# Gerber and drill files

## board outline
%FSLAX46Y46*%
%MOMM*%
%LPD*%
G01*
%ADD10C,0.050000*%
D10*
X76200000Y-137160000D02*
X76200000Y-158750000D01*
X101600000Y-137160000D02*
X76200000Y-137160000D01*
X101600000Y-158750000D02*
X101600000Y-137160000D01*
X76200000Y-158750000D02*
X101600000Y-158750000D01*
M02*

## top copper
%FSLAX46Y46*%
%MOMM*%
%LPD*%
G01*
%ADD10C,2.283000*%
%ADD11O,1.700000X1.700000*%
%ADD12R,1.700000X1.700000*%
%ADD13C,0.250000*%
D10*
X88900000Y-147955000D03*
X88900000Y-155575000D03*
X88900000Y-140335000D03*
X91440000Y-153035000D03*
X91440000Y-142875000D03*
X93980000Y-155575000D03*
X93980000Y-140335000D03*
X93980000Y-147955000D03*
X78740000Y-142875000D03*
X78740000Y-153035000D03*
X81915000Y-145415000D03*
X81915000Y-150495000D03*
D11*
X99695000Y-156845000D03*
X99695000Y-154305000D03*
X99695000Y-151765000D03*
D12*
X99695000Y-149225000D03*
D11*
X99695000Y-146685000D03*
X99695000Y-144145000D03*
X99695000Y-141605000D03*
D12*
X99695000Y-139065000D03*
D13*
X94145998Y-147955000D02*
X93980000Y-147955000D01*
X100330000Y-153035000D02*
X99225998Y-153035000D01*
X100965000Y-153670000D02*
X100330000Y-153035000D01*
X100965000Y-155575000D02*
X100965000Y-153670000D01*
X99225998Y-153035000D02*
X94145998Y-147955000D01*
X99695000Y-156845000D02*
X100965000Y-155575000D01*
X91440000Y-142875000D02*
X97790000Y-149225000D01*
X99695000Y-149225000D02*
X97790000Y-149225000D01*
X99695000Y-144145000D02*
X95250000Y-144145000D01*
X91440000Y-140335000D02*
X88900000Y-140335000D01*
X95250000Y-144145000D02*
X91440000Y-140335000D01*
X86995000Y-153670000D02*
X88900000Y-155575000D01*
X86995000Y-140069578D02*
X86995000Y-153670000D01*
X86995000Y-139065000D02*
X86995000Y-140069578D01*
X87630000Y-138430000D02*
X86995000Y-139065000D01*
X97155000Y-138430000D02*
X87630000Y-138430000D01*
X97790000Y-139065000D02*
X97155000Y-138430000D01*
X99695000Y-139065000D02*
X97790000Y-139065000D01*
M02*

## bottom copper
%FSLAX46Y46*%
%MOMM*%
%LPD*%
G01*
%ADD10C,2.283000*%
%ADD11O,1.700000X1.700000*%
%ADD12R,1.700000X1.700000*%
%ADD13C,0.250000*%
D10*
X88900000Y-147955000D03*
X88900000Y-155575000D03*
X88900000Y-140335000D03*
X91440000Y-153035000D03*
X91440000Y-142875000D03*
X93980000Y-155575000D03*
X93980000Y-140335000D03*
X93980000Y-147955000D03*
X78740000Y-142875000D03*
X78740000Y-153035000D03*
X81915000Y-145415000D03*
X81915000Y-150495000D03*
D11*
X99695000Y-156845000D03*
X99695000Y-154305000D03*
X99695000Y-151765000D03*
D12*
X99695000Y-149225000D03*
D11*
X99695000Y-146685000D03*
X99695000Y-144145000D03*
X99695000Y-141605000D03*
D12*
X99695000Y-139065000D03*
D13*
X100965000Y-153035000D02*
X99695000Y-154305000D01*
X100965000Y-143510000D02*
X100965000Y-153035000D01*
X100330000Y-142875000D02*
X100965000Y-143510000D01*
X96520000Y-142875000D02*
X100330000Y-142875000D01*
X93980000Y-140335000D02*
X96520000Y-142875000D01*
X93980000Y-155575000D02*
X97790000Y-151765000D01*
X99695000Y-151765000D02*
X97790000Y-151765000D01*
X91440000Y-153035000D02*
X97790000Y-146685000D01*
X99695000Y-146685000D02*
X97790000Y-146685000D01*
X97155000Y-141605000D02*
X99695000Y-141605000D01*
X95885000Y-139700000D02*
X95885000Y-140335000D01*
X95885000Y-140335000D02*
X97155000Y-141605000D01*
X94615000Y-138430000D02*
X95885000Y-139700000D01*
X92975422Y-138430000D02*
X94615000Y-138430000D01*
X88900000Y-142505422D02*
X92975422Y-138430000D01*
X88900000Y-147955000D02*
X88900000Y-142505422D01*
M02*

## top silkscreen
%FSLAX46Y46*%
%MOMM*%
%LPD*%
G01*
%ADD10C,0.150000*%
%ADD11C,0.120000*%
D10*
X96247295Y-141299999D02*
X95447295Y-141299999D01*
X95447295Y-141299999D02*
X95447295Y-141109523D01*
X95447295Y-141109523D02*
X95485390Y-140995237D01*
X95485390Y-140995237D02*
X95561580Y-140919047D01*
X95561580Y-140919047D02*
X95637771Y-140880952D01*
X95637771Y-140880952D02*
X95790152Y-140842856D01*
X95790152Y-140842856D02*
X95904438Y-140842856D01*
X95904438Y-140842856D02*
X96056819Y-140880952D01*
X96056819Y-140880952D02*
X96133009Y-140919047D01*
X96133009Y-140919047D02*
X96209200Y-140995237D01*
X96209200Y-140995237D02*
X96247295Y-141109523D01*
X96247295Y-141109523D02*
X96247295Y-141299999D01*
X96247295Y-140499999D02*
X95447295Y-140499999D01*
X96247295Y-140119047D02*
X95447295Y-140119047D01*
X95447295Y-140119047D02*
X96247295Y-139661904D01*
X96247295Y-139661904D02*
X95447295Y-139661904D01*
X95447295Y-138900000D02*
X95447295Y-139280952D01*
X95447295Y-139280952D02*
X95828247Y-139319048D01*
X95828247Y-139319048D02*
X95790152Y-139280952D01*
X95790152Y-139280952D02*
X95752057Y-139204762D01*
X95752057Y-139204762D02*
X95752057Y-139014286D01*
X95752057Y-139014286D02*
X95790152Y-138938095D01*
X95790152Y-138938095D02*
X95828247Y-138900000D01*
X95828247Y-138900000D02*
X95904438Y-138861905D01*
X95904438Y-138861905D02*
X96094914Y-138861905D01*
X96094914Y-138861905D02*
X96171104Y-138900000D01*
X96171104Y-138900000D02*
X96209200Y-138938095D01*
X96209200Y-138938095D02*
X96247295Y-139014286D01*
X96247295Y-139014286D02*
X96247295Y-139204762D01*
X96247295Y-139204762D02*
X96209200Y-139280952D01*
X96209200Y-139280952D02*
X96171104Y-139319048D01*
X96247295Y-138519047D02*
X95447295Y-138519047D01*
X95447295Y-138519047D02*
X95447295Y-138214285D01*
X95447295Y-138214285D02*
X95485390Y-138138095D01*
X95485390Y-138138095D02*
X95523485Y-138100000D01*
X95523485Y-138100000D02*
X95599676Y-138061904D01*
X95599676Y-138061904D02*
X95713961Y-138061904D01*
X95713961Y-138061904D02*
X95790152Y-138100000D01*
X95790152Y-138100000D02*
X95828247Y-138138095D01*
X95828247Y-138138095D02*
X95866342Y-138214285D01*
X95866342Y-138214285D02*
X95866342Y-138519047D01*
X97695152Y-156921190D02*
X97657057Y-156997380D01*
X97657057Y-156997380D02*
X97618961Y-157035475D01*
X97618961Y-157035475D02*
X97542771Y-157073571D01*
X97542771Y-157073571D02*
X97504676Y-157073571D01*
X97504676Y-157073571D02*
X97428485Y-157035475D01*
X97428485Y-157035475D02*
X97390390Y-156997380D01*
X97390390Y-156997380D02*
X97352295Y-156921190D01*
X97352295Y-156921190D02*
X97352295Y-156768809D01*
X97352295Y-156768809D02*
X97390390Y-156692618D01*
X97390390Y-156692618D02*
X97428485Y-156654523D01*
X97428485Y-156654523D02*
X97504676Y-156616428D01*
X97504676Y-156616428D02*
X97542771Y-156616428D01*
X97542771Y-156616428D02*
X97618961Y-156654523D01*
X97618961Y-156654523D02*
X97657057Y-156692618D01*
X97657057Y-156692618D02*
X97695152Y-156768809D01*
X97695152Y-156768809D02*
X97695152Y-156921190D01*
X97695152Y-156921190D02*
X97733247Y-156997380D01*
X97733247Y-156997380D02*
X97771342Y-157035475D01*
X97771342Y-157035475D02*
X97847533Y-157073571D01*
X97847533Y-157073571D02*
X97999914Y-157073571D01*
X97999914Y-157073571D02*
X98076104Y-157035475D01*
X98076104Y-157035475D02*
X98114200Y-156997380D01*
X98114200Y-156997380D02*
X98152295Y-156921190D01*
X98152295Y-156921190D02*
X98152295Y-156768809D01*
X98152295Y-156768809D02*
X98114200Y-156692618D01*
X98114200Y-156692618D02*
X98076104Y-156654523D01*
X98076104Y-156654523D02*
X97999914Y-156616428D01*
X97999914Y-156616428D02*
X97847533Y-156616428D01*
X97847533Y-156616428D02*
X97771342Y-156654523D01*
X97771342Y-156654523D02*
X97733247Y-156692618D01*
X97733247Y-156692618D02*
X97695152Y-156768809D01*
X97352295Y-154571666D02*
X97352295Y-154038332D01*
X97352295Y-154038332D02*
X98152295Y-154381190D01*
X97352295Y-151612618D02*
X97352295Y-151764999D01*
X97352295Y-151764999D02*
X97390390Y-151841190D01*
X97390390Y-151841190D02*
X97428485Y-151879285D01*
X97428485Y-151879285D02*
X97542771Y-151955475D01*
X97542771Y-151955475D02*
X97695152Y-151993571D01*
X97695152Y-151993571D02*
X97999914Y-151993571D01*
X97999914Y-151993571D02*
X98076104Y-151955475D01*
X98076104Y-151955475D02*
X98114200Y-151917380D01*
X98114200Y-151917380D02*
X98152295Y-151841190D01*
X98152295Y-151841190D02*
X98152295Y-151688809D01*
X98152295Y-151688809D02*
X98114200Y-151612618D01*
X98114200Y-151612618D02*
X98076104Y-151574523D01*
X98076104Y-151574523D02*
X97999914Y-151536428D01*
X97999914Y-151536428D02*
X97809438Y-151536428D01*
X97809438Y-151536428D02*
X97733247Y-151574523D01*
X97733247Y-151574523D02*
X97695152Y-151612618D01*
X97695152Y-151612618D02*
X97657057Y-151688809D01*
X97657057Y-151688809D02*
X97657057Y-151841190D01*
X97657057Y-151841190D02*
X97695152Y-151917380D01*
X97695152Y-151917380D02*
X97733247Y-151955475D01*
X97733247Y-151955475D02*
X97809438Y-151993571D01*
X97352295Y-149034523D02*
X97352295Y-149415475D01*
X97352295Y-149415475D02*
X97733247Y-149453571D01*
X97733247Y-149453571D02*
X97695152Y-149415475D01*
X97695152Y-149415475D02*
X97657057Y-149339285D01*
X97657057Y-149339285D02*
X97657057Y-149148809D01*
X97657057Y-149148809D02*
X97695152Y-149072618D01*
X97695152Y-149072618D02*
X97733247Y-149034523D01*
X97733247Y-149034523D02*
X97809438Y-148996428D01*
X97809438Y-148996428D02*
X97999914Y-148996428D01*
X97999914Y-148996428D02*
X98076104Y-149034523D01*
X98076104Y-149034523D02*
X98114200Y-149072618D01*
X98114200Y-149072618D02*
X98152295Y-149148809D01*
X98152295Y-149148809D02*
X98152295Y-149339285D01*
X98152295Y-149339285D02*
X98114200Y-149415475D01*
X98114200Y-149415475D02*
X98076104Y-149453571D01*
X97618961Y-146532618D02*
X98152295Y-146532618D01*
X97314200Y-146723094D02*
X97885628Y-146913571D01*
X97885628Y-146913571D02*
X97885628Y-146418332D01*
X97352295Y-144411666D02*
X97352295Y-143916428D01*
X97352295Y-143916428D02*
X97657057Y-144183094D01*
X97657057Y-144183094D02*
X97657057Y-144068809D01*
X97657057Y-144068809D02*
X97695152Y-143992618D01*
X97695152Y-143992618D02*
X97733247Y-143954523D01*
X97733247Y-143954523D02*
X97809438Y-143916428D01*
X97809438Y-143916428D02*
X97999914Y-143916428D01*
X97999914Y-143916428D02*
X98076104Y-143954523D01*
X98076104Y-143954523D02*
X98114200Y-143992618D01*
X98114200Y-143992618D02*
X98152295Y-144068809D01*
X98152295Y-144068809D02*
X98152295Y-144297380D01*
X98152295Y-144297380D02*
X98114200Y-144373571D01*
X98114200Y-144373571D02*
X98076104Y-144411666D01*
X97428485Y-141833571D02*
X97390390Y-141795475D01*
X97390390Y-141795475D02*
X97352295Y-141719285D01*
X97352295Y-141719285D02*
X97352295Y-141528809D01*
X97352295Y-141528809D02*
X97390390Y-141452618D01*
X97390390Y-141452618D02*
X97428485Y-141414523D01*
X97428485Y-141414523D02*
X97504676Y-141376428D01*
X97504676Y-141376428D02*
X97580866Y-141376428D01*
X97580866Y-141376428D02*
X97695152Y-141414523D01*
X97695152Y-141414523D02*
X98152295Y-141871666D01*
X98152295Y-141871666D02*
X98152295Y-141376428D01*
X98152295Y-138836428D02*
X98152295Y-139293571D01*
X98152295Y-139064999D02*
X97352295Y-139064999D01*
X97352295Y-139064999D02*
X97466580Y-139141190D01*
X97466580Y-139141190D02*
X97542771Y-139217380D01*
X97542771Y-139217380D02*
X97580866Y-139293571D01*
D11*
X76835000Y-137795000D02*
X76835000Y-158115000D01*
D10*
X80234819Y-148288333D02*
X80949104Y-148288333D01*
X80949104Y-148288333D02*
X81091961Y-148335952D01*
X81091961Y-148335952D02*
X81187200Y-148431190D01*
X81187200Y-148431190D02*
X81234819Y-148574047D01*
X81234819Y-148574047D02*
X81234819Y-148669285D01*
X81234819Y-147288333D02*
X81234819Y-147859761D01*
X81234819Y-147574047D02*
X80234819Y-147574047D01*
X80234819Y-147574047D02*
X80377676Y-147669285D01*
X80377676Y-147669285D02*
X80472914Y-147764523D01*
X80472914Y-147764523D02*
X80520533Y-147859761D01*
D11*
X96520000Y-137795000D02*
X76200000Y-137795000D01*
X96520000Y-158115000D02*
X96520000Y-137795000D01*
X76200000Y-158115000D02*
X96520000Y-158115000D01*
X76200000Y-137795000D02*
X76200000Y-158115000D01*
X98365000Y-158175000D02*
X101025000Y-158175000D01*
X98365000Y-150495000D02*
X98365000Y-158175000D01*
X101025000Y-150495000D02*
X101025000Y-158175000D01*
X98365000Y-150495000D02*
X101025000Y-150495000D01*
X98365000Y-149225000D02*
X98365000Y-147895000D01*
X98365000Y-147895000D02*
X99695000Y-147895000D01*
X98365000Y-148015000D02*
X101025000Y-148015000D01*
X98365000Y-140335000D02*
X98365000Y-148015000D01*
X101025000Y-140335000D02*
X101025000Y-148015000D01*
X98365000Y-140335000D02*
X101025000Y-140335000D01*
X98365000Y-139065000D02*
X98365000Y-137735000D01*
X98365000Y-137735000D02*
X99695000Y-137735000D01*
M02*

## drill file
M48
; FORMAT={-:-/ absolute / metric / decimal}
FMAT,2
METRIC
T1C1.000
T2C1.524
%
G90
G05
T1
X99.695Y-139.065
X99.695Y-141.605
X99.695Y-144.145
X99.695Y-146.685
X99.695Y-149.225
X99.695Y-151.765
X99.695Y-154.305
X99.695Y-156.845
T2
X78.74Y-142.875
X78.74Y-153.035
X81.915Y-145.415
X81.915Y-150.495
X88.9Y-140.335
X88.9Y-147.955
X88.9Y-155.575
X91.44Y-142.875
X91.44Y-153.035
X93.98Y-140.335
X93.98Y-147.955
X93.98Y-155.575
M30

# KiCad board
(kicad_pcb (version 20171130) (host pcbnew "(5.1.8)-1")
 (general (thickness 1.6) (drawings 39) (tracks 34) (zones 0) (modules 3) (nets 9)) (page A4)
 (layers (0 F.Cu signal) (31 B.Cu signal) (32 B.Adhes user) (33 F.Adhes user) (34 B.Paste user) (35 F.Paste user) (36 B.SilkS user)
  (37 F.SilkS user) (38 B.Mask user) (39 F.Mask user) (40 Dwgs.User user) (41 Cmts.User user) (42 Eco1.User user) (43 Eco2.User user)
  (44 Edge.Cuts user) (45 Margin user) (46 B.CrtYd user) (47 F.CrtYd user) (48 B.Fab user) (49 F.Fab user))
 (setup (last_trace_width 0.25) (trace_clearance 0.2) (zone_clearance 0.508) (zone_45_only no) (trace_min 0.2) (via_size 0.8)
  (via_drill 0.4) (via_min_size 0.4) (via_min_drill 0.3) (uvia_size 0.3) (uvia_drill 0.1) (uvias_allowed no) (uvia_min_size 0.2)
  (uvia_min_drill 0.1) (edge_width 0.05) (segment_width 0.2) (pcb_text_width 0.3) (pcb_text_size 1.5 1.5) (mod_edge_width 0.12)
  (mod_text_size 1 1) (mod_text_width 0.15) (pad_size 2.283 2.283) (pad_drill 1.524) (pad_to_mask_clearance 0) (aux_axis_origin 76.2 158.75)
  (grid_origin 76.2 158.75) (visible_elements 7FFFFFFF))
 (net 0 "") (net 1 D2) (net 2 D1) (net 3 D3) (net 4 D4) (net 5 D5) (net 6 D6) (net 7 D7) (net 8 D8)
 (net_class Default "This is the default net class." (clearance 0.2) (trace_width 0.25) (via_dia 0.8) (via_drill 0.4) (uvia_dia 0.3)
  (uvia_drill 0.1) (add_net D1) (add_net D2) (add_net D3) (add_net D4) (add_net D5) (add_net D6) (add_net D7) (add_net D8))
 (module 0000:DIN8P (layer F.Cu) (at 81.28 147.955 270)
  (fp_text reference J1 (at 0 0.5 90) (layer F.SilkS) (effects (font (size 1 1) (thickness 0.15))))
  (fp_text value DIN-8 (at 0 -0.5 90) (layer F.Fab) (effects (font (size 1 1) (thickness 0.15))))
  (fp_line (start -10.16 -15.24) (end -10.16 5.08) (layer F.SilkS) (width 0.12))
  (fp_line (start 10.16 -15.24) (end -10.16 -15.24) (layer F.SilkS) (width 0.12))
  (fp_line (start 10.16 5.08) (end 10.16 -15.24) (layer F.SilkS) (width 0.12))
  (fp_line (start -10.16 5.08) (end 10.16 5.08) (layer F.SilkS) (width 0.12))
  (pad 2 thru_hole circle (at 0 -7.62 270) (size 2.283 2.283) (drill 1.524) (layers *.Cu *.Mask) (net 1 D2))
  (pad 1 thru_hole circle (at 7.62 -7.62 270) (size 2.283 2.283) (drill 1.524) (layers *.Cu *.Mask) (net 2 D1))
  (pad 3 thru_hole circle (at -7.62 -7.62 270) (size 2.283 2.283) (drill 1.524) (layers *.Cu *.Mask) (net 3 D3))
  (pad 4 thru_hole circle (at 5.08 -10.16 270) (size 2.283 2.283) (drill 1.524) (layers *.Cu *.Mask) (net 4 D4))
  (pad 5 thru_hole circle (at -5.08 -10.16 270) (size 2.283 2.283) (drill 1.524) (layers *.Cu *.Mask) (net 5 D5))
  (pad 6 thru_hole circle (at 7.62 -12.7 270) (size 2.283 2.283) (drill 1.524) (layers *.Cu *.Mask) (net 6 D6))
  (pad 7 thru_hole circle (at -7.62 -12.7 270) (size 2.283 2.283) (drill 1.524) (layers *.Cu *.Mask) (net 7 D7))
  (pad 8 thru_hole circle (at 0 -12.7 270) (size 2.283 2.283) (drill 1.524) (layers *.Cu *.Mask) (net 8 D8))
  (pad "" thru_hole circle (at -5.08 2.54 270) (size 2.283 2.283) (drill 1.524) (layers *.Cu *.Mask))
  (pad "" thru_hole circle (at 5.08 2.54 270) (size 2.283 2.283) (drill 1.524) (layers *.Cu *.Mask))
  (pad "" thru_hole circle (at -2.54 -0.635 270) (size 2.283 2.283) (drill 1.524) (layers *.Cu *.Mask))
  (pad "" thru_hole circle (at 2.54 -0.635 270) (size 2.283 2.283) (drill 1.524) (layers *.Cu *.Mask)))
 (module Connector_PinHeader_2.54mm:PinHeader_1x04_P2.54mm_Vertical (layer F.Cu) (at 99.695 149.225)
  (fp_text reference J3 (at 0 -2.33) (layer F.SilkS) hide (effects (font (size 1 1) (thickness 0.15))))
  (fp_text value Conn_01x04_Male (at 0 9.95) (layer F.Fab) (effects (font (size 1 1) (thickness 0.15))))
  (fp_line (start -1.33 8.95) (end 1.33 8.95) (layer F.SilkS) (width 0.12))
  (fp_line (start -1.33 1.27) (end -1.33 8.95) (layer F.SilkS) (width 0.12))
  (fp_line (start 1.33 1.27) (end 1.33 8.95) (layer F.SilkS) (width 0.12))
  (fp_line (start -1.33 1.27) (end 1.33 1.27) (layer F.SilkS) (width 0.12))
  (fp_line (start -1.33 0) (end -1.33 -1.33) (layer F.SilkS) (width 0.12))
  (fp_line (start -1.33 -1.33) (end 0 -1.33) (layer F.SilkS) (width 0.12))
  (pad 4 thru_hole oval (at 0 7.62) (size 1.7 1.7) (drill 1) (layers *.Cu *.Mask) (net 8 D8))
  (pad 3 thru_hole oval (at 0 5.08) (size 1.7 1.7) (drill 1) (layers *.Cu *.Mask) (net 7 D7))
  (pad 2 thru_hole oval (at 0 2.54) (size 1.7 1.7) (drill 1) (layers *.Cu *.Mask) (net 6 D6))
  (pad 1 thru_hole rect (at 0 0) (size 1.7 1.7) (drill 1) (layers *.Cu *.Mask) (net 5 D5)))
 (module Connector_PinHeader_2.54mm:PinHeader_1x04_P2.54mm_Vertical (layer F.Cu) (at 99.695 139.065)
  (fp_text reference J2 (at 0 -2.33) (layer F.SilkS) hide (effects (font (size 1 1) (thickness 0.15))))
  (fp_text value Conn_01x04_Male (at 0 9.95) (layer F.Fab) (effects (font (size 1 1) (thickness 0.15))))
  (fp_line (start -1.33 8.95) (end 1.33 8.95) (layer F.SilkS) (width 0.12))
  (fp_line (start -1.33 1.27) (end -1.33 8.95) (layer F.SilkS) (width 0.12))
  (fp_line (start 1.33 1.27) (end 1.33 8.95) (layer F.SilkS) (width 0.12))
  (fp_line (start -1.33 1.27) (end 1.33 1.27) (layer F.SilkS) (width 0.12))
  (fp_line (start -1.33 0) (end -1.33 -1.33) (layer F.SilkS) (width 0.12))
  (fp_line (start -1.33 -1.33) (end 0 -1.33) (layer F.SilkS) (width 0.12))
  (pad 4 thru_hole oval (at 0 7.62) (size 1.7 1.7) (drill 1) (layers *.Cu *.Mask) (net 4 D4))
  (pad 3 thru_hole oval (at 0 5.08) (size 1.7 1.7) (drill 1) (layers *.Cu *.Mask) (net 3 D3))
  (pad 2 thru_hole oval (at 0 2.54) (size 1.7 1.7) (drill 1) (layers *.Cu *.Mask) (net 1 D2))
  (pad 1 thru_hole rect (at 0 0) (size 1.7 1.7) (drill 1) (layers *.Cu *.Mask) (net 2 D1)))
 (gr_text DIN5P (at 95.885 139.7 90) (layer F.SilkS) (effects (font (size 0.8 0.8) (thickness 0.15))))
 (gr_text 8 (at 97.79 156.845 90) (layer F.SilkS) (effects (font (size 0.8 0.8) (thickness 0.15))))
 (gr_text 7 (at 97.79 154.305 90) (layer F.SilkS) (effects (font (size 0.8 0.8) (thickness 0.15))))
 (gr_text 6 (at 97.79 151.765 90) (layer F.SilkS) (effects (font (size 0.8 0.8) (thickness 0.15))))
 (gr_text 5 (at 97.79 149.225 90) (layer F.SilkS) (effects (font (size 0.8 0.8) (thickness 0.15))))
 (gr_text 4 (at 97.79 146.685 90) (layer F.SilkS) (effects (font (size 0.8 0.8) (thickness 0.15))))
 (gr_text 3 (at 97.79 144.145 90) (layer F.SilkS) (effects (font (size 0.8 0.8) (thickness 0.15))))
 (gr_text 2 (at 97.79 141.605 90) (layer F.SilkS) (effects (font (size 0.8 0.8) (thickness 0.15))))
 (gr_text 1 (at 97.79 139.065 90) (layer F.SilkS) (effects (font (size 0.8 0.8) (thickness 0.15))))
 (gr_line (start 76.2 137.16) (end 76.2 158.75) (layer Edge.Cuts) (width 0.05))
 (gr_line (start 101.6 137.16) (end 76.2 137.16) (layer Edge.Cuts) (width 0.05))
 (gr_line (start 101.6 158.75) (end 101.6 137.16) (layer Edge.Cuts) (width 0.05))
 (gr_line (start 76.2 158.75) (end 101.6 158.75) (layer Edge.Cuts) (width 0.05))
 (gr_line (start 76.835 137.795) (end 76.835 158.115) (layer F.SilkS) (width 0.12))
 (segment (start 94.145998 147.955) (end 93.98 147.955) (width 0.25) (layer F.Cu) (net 8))
 (segment (start 100.33 153.035) (end 99.225998 153.035) (width 0.25) (layer F.Cu) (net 8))
 (segment (start 100.965 153.67) (end 100.33 153.035) (width 0.25) (layer F.Cu) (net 8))
 (segment (start 100.965 155.575) (end 100.965 153.67) (width 0.25) (layer F.Cu) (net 8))
 (segment (start 99.225998 153.035) (end 94.145998 147.955) (width 0.25) (layer F.Cu) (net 8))
 (segment (start 99.695 156.845) (end 100.965 155.575) (width 0.25) (layer F.Cu) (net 8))
 (segment (start 100.965 153.035) (end 99.695 154.305) (width 0.25) (layer B.Cu) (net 7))
 (segment (start 100.965 143.51) (end 100.965 153.035) (width 0.25) (layer B.Cu) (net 7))
 (segment (start 100.33 142.875) (end 100.965 143.51) (width 0.25) (layer B.Cu) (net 7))
 (segment (start 96.52 142.875) (end 100.33 142.875) (width 0.25) (layer B.Cu) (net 7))
 (segment (start 93.98 140.335) (end 96.52 142.875) (width 0.25) (layer B.Cu) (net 7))
 (segment (start 93.98 155.575) (end 97.79 151.765) (width 0.25) (layer B.Cu) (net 6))
 (segment (start 99.695 151.765) (end 97.79 151.765) (width 0.25) (layer B.Cu) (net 6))
 (segment (start 91.44 142.875) (end 97.79 149.225) (width 0.25) (layer F.Cu) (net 5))
 (segment (start 99.695 149.225) (end 97.79 149.225) (width 0.25) (layer F.Cu) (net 5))
 (segment (start 91.44 153.035) (end 97.79 146.685) (width 0.25) (layer B.Cu) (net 4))
 (segment (start 99.695 146.685) (end 97.79 146.685) (width 0.25) (layer B.Cu) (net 4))
 (segment (start 99.695 144.145) (end 95.25 144.145) (width 0.25) (layer F.Cu) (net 3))
 (segment (start 91.44 140.335) (end 88.9 140.335) (width 0.25) (layer F.Cu) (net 3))
 (segment (start 95.25 144.145) (end 91.44 140.335) (width 0.25) (layer F.Cu) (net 3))
 (segment (start 86.995 153.67) (end 88.9 155.575) (width 0.25) (layer F.Cu) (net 2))
 (segment (start 86.995 140.069578) (end 86.995 153.67) (width 0.25) (layer F.Cu) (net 2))
 (segment (start 86.995 139.065) (end 86.995 140.069578) (width 0.25) (layer F.Cu) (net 2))
 (segment (start 87.63 138.43) (end 86.995 139.065) (width 0.25) (layer F.Cu) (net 2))
 (segment (start 97.155 138.43) (end 87.63 138.43) (width 0.25) (layer F.Cu) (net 2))
 (segment (start 97.79 139.065) (end 97.155 138.43) (width 0.25) (layer F.Cu) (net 2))
 (segment (start 99.695 139.065) (end 97.79 139.065) (width 0.25) (layer F.Cu) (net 2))
 (segment (start 97.155 141.605) (end 99.695 141.605) (width 0.25) (layer B.Cu) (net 1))
 (segment (start 95.885 139.7) (end 95.885 140.335) (width 0.25) (layer B.Cu) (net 1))
 (segment (start 95.885 140.335) (end 97.155 141.605) (width 0.25) (layer B.Cu) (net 1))
 (segment (start 94.615 138.43) (end 95.885 139.7) (width 0.25) (layer B.Cu) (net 1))
 (segment (start 92.975422 138.43) (end 94.615 138.43) (width 0.25) (layer B.Cu) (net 1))
 (segment (start 88.9 142.505422) (end 92.975422 138.43) (width 0.25) (layer B.Cu) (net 1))
 (segment (start 88.9 147.955) (end 88.9 142.505422) (width 0.25) (layer B.Cu) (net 1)))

